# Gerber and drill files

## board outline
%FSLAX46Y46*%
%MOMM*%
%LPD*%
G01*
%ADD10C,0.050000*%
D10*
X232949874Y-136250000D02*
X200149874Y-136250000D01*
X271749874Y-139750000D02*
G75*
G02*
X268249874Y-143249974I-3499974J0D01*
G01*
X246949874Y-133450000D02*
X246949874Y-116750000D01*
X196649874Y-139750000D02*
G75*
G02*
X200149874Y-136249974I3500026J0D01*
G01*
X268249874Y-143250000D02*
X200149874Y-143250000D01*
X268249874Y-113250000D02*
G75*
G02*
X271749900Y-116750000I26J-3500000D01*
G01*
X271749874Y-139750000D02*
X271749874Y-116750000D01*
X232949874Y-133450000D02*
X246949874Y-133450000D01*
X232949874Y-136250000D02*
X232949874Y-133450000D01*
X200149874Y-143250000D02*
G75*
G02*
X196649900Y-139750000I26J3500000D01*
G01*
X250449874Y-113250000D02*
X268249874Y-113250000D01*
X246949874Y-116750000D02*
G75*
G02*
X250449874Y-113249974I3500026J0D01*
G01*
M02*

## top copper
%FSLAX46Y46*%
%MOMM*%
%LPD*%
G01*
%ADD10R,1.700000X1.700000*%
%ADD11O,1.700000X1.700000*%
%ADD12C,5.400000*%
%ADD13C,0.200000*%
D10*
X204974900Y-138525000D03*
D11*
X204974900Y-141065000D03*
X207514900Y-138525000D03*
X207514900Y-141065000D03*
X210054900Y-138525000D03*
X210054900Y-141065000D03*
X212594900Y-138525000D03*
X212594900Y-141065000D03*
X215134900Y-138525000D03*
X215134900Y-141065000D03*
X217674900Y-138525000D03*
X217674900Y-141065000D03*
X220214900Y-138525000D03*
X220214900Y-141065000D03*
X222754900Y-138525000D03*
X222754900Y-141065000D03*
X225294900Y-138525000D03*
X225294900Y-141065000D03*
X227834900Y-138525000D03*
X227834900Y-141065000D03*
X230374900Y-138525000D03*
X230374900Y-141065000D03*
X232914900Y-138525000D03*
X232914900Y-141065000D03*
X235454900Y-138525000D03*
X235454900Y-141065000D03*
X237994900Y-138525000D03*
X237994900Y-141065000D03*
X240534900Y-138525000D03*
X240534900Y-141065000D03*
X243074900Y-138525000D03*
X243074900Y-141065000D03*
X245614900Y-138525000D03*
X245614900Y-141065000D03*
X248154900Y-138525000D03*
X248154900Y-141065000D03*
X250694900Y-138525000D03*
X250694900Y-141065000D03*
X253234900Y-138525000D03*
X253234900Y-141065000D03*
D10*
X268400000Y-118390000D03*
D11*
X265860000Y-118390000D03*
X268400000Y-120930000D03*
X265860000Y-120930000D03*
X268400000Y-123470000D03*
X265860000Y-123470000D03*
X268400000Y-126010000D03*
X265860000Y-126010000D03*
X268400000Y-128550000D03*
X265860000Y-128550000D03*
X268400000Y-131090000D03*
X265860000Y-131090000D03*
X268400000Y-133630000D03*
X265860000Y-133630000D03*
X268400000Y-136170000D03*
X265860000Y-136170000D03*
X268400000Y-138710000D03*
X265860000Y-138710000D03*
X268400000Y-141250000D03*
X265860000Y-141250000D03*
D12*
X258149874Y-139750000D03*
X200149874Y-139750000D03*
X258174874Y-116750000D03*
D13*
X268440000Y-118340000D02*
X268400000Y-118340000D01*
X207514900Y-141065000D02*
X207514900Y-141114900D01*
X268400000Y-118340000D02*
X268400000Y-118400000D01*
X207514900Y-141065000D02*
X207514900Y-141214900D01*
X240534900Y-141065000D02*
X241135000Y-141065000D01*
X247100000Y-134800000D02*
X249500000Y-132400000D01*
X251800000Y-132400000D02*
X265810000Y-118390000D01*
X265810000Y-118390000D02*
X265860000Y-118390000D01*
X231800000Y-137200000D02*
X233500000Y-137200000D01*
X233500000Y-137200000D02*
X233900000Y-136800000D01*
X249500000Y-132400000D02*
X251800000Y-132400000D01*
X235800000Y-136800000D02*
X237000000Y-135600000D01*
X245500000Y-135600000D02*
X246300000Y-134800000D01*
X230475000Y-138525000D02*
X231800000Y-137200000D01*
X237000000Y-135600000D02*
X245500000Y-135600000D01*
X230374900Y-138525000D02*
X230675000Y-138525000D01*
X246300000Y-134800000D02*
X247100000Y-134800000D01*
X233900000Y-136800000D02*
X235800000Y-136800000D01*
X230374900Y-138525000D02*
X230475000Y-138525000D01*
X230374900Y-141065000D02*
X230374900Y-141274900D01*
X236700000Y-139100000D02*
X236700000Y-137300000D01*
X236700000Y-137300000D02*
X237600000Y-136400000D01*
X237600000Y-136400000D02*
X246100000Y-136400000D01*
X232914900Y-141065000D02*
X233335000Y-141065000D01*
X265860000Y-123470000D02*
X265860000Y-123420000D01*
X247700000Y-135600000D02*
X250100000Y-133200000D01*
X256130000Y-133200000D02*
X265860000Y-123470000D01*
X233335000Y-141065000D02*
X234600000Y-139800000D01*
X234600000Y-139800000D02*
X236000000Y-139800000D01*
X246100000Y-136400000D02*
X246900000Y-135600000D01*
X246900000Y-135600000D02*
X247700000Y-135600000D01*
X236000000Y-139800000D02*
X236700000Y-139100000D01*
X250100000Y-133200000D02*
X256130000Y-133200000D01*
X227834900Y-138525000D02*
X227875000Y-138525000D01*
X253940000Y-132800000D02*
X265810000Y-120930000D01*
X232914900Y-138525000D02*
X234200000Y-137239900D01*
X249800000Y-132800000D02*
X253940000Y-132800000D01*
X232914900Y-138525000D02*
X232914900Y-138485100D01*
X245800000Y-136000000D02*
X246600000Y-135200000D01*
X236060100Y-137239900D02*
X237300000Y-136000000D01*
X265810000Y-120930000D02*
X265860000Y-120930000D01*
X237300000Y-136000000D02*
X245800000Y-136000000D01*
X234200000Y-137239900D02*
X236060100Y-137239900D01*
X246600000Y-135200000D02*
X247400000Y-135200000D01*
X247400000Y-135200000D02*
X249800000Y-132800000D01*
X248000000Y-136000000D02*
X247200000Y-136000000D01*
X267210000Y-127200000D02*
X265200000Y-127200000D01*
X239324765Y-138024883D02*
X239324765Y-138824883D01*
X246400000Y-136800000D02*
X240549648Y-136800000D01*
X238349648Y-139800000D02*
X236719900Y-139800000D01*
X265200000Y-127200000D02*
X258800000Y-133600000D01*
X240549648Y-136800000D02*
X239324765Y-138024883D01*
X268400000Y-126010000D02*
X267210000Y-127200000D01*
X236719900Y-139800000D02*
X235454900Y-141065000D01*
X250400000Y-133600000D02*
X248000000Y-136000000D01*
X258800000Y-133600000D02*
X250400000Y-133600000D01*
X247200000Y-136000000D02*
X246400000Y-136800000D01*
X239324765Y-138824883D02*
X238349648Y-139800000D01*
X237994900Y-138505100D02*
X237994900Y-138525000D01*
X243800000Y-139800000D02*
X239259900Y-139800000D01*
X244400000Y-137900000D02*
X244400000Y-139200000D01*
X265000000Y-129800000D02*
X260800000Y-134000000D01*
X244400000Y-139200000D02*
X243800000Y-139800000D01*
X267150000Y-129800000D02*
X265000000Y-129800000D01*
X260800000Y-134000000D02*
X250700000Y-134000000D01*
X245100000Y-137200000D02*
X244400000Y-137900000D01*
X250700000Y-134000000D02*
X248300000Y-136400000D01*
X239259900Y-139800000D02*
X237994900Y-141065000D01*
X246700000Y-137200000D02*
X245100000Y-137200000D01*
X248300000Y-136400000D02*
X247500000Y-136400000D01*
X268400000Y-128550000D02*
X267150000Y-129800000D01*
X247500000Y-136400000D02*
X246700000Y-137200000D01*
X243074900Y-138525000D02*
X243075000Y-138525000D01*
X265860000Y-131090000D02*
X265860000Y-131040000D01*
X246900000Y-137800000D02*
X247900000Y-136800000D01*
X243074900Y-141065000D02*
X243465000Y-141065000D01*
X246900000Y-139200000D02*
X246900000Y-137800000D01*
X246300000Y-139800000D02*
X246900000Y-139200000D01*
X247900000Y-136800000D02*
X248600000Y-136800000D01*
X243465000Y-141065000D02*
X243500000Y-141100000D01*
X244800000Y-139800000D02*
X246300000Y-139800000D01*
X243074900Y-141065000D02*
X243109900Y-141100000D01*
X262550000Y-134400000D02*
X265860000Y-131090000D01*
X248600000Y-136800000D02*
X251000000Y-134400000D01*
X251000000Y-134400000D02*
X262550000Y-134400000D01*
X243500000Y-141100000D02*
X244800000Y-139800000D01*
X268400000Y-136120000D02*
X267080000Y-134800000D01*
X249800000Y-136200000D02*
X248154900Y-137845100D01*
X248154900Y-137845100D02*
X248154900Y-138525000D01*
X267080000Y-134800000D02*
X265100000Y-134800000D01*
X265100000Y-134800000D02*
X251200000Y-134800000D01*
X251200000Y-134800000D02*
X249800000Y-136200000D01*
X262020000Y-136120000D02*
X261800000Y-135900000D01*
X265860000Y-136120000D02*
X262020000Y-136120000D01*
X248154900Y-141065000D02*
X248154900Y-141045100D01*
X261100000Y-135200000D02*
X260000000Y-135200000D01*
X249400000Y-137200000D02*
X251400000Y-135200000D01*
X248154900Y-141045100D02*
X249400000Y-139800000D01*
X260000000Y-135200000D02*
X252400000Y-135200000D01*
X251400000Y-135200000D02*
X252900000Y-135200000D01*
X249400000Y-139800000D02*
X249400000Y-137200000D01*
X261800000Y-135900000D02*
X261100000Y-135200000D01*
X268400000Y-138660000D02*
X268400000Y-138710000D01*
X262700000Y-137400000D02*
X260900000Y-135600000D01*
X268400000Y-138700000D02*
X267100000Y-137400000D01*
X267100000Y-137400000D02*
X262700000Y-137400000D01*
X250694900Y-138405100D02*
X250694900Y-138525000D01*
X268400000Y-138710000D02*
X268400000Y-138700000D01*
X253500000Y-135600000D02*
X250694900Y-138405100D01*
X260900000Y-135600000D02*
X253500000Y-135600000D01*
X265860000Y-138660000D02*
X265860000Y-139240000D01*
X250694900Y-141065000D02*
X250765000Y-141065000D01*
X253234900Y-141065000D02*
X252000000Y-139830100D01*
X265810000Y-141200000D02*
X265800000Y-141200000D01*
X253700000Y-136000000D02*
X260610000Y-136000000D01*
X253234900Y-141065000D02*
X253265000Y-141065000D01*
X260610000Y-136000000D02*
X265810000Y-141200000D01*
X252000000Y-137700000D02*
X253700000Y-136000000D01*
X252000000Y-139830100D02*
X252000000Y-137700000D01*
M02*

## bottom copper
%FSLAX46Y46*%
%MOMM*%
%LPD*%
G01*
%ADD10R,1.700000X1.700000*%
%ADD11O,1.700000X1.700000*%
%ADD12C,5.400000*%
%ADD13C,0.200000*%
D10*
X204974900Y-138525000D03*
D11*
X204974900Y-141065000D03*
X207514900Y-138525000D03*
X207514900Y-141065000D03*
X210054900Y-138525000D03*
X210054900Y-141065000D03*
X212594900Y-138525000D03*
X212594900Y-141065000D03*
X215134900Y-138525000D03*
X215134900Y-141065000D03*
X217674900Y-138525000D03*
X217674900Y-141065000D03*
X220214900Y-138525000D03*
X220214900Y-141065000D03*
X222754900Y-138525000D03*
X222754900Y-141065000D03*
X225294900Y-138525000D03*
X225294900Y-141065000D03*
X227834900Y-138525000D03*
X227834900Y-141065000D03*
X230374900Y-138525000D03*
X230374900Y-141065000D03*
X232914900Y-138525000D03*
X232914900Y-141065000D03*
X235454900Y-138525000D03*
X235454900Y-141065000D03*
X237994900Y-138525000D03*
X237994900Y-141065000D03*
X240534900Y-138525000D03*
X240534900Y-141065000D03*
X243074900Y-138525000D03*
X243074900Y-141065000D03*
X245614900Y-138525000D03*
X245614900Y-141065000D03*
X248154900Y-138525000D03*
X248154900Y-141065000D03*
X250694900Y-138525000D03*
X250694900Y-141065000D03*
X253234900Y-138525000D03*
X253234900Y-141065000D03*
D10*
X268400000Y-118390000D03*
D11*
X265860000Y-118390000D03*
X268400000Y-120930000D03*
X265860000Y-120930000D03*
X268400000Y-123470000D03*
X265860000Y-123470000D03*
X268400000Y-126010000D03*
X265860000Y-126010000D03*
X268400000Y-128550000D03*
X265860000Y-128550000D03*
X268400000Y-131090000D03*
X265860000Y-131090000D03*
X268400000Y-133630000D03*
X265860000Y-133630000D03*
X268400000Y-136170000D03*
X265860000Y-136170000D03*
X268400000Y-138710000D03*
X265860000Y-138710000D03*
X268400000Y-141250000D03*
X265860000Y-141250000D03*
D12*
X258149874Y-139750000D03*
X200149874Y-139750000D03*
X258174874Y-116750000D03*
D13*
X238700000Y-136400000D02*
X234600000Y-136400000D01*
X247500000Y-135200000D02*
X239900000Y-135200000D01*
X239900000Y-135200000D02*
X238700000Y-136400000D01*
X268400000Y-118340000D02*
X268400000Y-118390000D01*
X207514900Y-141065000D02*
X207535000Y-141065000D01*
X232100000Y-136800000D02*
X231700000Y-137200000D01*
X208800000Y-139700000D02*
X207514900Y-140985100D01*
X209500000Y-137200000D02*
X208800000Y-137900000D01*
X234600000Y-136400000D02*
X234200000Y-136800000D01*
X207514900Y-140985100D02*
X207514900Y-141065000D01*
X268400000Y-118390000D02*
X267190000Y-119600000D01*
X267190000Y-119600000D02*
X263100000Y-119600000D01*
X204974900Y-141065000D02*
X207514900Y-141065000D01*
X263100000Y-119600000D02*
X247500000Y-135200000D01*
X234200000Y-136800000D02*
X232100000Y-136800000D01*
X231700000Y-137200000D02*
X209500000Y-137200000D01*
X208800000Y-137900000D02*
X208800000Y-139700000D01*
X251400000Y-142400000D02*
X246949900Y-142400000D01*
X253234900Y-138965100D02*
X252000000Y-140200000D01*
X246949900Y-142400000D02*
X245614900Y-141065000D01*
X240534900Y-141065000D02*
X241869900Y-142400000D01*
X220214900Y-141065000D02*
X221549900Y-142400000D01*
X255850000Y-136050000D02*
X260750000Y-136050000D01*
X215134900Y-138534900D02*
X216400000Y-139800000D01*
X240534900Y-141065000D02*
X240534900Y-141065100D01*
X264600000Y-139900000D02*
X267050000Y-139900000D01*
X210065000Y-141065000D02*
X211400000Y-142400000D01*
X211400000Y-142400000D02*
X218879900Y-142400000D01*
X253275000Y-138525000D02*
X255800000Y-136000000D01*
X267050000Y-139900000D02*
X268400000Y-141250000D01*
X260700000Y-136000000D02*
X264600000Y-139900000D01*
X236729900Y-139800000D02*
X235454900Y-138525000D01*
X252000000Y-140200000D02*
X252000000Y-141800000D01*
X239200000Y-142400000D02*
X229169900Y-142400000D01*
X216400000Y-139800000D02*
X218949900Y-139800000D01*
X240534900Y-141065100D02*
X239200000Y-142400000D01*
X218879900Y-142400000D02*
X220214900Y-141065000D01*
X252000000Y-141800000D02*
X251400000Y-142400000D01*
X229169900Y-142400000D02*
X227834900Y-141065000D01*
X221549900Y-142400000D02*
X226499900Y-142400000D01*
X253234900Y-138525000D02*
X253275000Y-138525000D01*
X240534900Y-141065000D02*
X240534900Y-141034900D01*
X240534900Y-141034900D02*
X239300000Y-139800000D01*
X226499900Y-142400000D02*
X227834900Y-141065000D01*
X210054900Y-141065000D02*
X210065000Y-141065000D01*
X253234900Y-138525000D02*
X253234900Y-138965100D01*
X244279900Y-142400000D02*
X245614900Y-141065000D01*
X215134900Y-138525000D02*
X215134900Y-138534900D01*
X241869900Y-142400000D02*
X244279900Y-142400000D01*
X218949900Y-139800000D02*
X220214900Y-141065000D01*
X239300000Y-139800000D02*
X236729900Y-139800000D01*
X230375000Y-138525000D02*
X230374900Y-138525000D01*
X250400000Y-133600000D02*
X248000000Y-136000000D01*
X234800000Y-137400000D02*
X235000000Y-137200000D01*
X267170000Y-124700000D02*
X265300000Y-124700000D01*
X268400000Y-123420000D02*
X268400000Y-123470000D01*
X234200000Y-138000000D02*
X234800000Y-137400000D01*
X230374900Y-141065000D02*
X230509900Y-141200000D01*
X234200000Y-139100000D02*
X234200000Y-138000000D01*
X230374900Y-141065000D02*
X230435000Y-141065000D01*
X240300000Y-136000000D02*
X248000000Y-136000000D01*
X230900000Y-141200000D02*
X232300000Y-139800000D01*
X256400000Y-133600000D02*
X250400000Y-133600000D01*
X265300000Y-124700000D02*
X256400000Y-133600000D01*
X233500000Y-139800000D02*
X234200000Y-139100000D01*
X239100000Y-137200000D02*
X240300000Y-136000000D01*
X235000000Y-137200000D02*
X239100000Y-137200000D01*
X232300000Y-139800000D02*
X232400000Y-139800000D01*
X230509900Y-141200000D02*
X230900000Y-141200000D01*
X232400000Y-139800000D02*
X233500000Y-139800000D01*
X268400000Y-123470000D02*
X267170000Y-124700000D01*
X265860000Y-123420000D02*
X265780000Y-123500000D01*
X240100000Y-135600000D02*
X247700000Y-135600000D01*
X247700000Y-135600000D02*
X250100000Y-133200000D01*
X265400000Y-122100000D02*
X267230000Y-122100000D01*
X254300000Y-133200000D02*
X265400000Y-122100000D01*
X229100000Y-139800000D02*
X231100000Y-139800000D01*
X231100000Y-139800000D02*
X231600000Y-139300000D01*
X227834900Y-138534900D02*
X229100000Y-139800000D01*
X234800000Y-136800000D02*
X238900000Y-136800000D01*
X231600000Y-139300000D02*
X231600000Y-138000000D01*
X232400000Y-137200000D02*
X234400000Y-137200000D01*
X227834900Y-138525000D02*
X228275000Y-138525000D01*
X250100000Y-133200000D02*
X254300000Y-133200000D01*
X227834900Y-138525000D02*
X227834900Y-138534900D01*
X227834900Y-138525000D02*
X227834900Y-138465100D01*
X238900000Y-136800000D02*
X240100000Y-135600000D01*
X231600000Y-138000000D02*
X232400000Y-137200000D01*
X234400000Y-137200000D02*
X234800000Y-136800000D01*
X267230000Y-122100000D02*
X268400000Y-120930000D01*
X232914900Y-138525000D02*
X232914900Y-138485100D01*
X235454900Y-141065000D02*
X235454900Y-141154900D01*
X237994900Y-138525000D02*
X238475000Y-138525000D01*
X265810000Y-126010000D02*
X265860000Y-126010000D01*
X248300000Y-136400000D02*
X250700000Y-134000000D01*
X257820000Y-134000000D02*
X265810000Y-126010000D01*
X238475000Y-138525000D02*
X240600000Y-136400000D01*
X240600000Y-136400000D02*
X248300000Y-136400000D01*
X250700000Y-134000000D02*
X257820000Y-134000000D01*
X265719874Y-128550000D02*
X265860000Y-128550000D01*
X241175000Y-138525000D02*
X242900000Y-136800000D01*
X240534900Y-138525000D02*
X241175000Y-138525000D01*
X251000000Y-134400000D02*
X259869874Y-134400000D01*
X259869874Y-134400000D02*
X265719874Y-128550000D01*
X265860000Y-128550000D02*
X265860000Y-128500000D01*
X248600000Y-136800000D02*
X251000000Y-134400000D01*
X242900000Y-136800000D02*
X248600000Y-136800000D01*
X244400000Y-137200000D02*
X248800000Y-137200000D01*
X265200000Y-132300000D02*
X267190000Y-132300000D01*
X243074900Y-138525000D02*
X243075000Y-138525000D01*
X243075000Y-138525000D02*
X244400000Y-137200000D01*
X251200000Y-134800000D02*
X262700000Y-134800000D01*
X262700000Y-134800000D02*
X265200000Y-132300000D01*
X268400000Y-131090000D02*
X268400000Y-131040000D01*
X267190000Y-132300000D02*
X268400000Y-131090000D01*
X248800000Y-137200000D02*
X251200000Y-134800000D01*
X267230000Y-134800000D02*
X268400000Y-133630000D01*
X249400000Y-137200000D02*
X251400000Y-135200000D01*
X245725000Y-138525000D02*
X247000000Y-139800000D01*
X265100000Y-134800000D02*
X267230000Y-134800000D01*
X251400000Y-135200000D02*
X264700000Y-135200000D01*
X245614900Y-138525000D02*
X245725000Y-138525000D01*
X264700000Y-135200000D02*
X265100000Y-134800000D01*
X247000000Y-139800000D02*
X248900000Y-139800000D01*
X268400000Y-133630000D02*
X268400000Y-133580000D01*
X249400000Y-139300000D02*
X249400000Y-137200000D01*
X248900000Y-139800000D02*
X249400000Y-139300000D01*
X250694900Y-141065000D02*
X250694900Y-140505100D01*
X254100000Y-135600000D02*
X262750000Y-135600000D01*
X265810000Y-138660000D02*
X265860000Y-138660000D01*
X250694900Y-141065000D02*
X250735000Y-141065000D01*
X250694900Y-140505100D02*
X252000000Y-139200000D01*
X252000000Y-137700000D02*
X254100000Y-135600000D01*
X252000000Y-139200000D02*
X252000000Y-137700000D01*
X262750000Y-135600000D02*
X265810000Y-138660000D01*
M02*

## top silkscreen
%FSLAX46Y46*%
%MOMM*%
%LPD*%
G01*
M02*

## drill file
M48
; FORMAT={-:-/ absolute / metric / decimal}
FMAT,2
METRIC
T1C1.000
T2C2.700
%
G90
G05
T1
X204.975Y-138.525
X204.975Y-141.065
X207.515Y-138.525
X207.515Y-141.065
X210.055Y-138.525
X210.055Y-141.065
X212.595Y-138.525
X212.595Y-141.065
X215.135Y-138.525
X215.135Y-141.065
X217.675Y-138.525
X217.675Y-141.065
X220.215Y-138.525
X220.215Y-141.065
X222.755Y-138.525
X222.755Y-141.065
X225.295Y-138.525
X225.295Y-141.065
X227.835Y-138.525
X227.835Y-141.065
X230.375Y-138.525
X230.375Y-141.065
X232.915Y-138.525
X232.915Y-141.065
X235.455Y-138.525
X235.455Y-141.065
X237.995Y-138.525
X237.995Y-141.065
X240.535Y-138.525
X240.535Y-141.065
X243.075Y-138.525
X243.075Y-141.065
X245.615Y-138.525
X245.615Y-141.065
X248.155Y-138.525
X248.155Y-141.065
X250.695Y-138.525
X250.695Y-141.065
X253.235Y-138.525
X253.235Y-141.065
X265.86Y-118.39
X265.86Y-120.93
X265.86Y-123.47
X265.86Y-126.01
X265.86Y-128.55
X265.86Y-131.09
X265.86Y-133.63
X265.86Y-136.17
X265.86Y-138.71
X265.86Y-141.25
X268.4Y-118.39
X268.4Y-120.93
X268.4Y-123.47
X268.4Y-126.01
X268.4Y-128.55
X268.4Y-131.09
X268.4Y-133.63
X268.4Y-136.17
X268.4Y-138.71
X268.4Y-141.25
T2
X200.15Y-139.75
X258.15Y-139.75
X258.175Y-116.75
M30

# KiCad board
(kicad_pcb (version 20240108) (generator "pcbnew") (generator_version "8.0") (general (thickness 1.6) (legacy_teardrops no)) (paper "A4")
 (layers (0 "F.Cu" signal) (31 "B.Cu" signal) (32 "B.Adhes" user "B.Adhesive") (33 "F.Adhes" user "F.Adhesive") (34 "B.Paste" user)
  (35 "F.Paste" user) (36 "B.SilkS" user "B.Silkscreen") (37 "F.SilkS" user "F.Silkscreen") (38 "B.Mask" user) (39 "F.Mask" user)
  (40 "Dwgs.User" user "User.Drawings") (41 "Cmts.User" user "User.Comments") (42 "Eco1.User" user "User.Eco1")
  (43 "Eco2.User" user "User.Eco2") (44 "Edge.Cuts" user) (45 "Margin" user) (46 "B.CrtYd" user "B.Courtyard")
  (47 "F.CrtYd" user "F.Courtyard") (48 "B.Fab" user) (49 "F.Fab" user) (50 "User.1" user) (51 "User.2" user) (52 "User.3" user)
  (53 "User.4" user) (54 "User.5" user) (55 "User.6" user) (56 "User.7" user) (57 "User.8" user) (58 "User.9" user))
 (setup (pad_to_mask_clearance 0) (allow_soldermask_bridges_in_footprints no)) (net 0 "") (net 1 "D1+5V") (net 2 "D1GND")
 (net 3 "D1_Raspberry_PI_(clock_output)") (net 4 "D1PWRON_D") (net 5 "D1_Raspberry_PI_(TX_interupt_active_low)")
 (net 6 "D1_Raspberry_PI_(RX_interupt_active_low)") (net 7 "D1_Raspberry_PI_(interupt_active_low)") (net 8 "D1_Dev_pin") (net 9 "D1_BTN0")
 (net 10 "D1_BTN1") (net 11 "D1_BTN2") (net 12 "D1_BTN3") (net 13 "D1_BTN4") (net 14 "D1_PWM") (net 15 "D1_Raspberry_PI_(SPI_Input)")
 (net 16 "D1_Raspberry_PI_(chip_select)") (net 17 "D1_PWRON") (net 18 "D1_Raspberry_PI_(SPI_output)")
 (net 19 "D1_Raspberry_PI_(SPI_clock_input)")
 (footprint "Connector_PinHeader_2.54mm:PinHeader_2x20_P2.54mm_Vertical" (layer "B.Cu") (at 204.9749 138.525 -90)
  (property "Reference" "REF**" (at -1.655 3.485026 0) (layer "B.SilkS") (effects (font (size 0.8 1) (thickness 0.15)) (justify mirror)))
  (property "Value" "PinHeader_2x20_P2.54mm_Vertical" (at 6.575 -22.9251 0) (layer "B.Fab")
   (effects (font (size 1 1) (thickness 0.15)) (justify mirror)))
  (pad "1" thru_hole rect (at 0 0 270) (size 1.7 1.7) (drill 1) (layers "*.Cu" "*.Mask") (remove_unused_layers no))
  (pad "2" thru_hole oval (at 2.54 0 270) (size 1.7 1.7) (drill 1) (layers "*.Cu" "*.Mask") (remove_unused_layers no) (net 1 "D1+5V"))
  (pad "3" thru_hole oval (at 0 -2.54 270) (size 1.7 1.7) (drill 1) (layers "*.Cu" "*.Mask") (remove_unused_layers no))
  (pad "4" thru_hole oval (at 2.54 -2.54 270) (size 1.7 1.7) (drill 1) (layers "*.Cu" "*.Mask") (remove_unused_layers no) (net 1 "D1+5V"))
  (pad "5" thru_hole oval (at 0 -5.08 270) (size 1.7 1.7) (drill 1) (layers "*.Cu" "*.Mask") (remove_unused_layers no))
  (pad "6" thru_hole oval (at 2.54 -5.08 270) (size 1.7 1.7) (drill 1) (layers "*.Cu" "*.Mask") (remove_unused_layers no) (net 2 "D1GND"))
  (pad "7" thru_hole oval (at 0 -7.62 270) (size 1.7 1.7) (drill 1) (layers "*.Cu" "*.Mask") (remove_unused_layers no))
  (pad "8" thru_hole oval (at 2.54 -7.62 270) (size 1.7 1.7) (drill 1) (layers "*.Cu" "*.Mask") (remove_unused_layers no))
  (pad "9" thru_hole oval (at 0 -10.16 270) (size 1.7 1.7) (drill 1) (layers "*.Cu" "*.Mask") (remove_unused_layers no) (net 2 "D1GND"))
  (pad "10" thru_hole oval (at 2.54 -10.16 270) (size 1.7 1.7) (drill 1) (layers "*.Cu" "*.Mask") (remove_unused_layers no))
  (pad "11" thru_hole oval (at 0 -12.7 270) (size 1.7 1.7) (drill 1) (layers "*.Cu" "*.Mask") (remove_unused_layers no))
  (pad "12" thru_hole oval (at 2.54 -12.7 270) (size 1.7 1.7) (drill 1) (layers "*.Cu" "*.Mask") (remove_unused_layers no))
  (pad "13" thru_hole oval (at 0 -15.24 270) (size 1.7 1.7) (drill 1) (layers "*.Cu" "*.Mask") (remove_unused_layers no))
  (pad "14" thru_hole oval (at 2.54 -15.24 270) (size 1.7 1.7) (drill 1) (layers "*.Cu" "*.Mask") (remove_unused_layers no) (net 2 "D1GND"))
  (pad "15" thru_hole oval (at 0 -17.78 270) (size 1.7 1.7) (drill 1) (layers "*.Cu" "*.Mask") (remove_unused_layers no))
  (pad "16" thru_hole oval (at 2.54 -17.78 270) (size 1.7 1.7) (drill 1) (layers "*.Cu" "*.Mask") (remove_unused_layers no))
  (pad "17" thru_hole oval (at 0 -20.32 270) (size 1.7 1.7) (drill 1) (layers "*.Cu" "*.Mask") (remove_unused_layers no))
  (pad "18" thru_hole oval (at 2.54 -20.32 270) (size 1.7 1.7) (drill 1) (layers "*.Cu" "*.Mask") (remove_unused_layers no))
  (pad "19" thru_hole oval (at 0 -22.86 270) (size 1.7 1.7) (drill 1) (layers "*.Cu" "*.Mask") (remove_unused_layers no)
   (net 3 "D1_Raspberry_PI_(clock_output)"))
  (pad "20" thru_hole oval (at 2.54 -22.86 270) (size 1.7 1.7) (drill 1) (layers "*.Cu" "*.Mask") (remove_unused_layers no) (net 2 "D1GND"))
  (pad "21" thru_hole oval (at 0 -25.4 270) (size 1.7 1.7) (drill 1) (layers "*.Cu" "*.Mask") (remove_unused_layers no) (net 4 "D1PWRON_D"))
  (pad "22" thru_hole oval (at 2.54 -25.4 270) (size 1.7 1.7) (drill 1) (layers "*.Cu" "*.Mask") (remove_unused_layers no)
   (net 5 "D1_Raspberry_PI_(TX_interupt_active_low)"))
  (pad "23" thru_hole oval (at 0 -27.94 270) (size 1.7 1.7) (drill 1) (layers "*.Cu" "*.Mask") (remove_unused_layers no)
   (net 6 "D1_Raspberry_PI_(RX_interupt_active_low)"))
  (pad "24" thru_hole oval (at 2.54 -27.94 270) (size 1.7 1.7) (drill 1) (layers "*.Cu" "*.Mask") (remove_unused_layers no)
   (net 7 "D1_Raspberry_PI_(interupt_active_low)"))
  (pad "25" thru_hole oval (at 0 -30.48 270) (size 1.7 1.7) (drill 1) (layers "*.Cu" "*.Mask") (remove_unused_layers no) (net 2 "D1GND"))
  (pad "26" thru_hole oval (at 2.54 -30.48 270) (size 1.7 1.7) (drill 1) (layers "*.Cu" "*.Mask") (remove_unused_layers no)
   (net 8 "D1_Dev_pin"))
  (pad "27" thru_hole oval (at 0 -33.02 270) (size 1.7 1.7) (drill 1) (layers "*.Cu" "*.Mask") (remove_unused_layers no) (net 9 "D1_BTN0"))
  (pad "28" thru_hole oval (at 2.54 -33.02 270) (size 1.7 1.7) (drill 1) (layers "*.Cu" "*.Mask") (remove_unused_layers no)
   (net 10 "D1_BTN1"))
  (pad "29" thru_hole oval (at 0 -35.56 270) (size 1.7 1.7) (drill 1) (layers "*.Cu" "*.Mask") (remove_unused_layers no) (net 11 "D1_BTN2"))
  (pad "30" thru_hole oval (at 2.54 -35.56 270) (size 1.7 1.7) (drill 1) (layers "*.Cu" "*.Mask") (remove_unused_layers no) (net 2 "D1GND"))
  (pad "31" thru_hole oval (at 0 -38.1 270) (size 1.7 1.7) (drill 1) (layers "*.Cu" "*.Mask") (remove_unused_layers no) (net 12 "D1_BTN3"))
  (pad "32" thru_hole oval (at 2.54 -38.1 270) (size 1.7 1.7) (drill 1) (layers "*.Cu" "*.Mask") (remove_unused_layers no)
   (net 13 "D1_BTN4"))
  (pad "33" thru_hole oval (at 0 -40.64 270) (size 1.7 1.7) (drill 1) (layers "*.Cu" "*.Mask") (remove_unused_layers no) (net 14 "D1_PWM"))
  (pad "34" thru_hole oval (at 2.54 -40.64 270) (size 1.7 1.7) (drill 1) (layers "*.Cu" "*.Mask") (remove_unused_layers no) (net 2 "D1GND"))
  (pad "35" thru_hole oval (at 0 -43.18 270) (size 1.7 1.7) (drill 1) (layers "*.Cu" "*.Mask") (remove_unused_layers no)
   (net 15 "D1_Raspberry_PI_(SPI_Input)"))
  (pad "36" thru_hole oval (at 2.54 -43.18 270) (size 1.7 1.7) (drill 1) (layers "*.Cu" "*.Mask") (remove_unused_layers no)
   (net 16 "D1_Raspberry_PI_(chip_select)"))
  (pad "37" thru_hole oval (at 0 -45.72 270) (size 1.7 1.7) (drill 1) (layers "*.Cu" "*.Mask") (remove_unused_layers no) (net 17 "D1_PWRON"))
  (pad "38" thru_hole oval (at 2.54 -45.72 270) (size 1.7 1.7) (drill 1) (layers "*.Cu" "*.Mask") (remove_unused_layers no)
   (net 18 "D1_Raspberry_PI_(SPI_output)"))
  (pad "39" thru_hole oval (at 0 -48.26 270) (size 1.7 1.7) (drill 1) (layers "*.Cu" "*.Mask") (remove_unused_layers no) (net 2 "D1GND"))
  (pad "40" thru_hole oval (at 2.54 -48.26 270) (size 1.7 1.7) (drill 1) (layers "*.Cu" "*.Mask") (remove_unused_layers no)
   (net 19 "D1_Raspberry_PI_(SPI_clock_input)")))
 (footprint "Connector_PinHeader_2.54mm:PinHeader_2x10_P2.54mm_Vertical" (layer "B.Cu") (at 268.4 118.39 180)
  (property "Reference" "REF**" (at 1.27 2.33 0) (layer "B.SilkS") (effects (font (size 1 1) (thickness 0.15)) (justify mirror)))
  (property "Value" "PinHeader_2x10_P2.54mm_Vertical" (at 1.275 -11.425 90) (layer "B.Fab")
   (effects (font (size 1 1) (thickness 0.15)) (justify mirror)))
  (pad "1" thru_hole rect (at 0 0 180) (size 1.7 1.7) (drill 1) (layers "*.Cu" "*.Mask") (remove_unused_layers no) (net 1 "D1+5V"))
  (pad "2" thru_hole oval (at 2.54 0 180) (size 1.7 1.7) (drill 1) (layers "*.Cu" "*.Mask") (remove_unused_layers no) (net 4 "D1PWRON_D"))
  (pad "3" thru_hole oval (at 0 -2.54 180) (size 1.7 1.7) (drill 1) (layers "*.Cu" "*.Mask") (remove_unused_layers no)
   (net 3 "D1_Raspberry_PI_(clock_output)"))
  (pad "4" thru_hole oval (at 2.54 -2.54 180) (size 1.7 1.7) (drill 1) (layers "*.Cu" "*.Mask") (remove_unused_layers no)
   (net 6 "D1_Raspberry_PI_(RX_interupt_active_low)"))
  (pad "5" thru_hole oval (at 0 -5.08 180) (size 1.7 1.7) (drill 1) (layers "*.Cu" "*.Mask") (remove_unused_layers no)
   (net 5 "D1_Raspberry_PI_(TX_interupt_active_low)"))
  (pad "6" thru_hole oval (at 2.54 -5.08 180) (size 1.7 1.7) (drill 1) (layers "*.Cu" "*.Mask") (remove_unused_layers no)
   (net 7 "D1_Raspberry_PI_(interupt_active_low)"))
  (pad "7" thru_hole oval (at 0 -7.62 180) (size 1.7 1.7) (drill 1) (layers "*.Cu" "*.Mask") (remove_unused_layers no) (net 8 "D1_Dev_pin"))
  (pad "8" thru_hole oval (at 2.54 -7.62 180) (size 1.7 1.7) (drill 1) (layers "*.Cu" "*.Mask") (remove_unused_layers no) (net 9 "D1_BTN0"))
  (pad "9" thru_hole oval (at 0 -10.16 180) (size 1.7 1.7) (drill 1) (layers "*.Cu" "*.Mask") (remove_unused_layers no) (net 10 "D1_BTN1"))
  (pad "10" thru_hole oval (at 2.54 -10.16 180) (size 1.7 1.7) (drill 1) (layers "*.Cu" "*.Mask") (remove_unused_layers no)
   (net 11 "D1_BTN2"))
  (pad "11" thru_hole oval (at 0 -12.7 180) (size 1.7 1.7) (drill 1) (layers "*.Cu" "*.Mask") (remove_unused_layers no) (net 12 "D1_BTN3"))
  (pad "12" thru_hole oval (at 2.54 -12.7 180) (size 1.7 1.7) (drill 1) (layers "*.Cu" "*.Mask") (remove_unused_layers no)
   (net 13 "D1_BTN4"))
  (pad "13" thru_hole oval (at 0 -15.24 180) (size 1.7 1.7) (drill 1) (layers "*.Cu" "*.Mask") (remove_unused_layers no) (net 14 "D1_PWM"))
  (pad "14" thru_hole oval (at 2.54 -15.24 180) (size 1.7 1.7) (drill 1) (layers "*.Cu" "*.Mask") (remove_unused_layers no))
  (pad "15" thru_hole oval (at 0 -17.78 180) (size 1.7 1.7) (drill 1) (layers "*.Cu" "*.Mask") (remove_unused_layers no)
   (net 15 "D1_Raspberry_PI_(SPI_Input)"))
  (pad "16" thru_hole oval (at 2.54 -17.78 180) (size 1.7 1.7) (drill 1) (layers "*.Cu" "*.Mask") (remove_unused_layers no)
   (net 16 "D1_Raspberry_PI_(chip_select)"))
  (pad "17" thru_hole oval (at 0 -20.32 180) (size 1.7 1.7) (drill 1) (layers "*.Cu" "*.Mask") (remove_unused_layers no) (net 17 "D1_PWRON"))
  (pad "18" thru_hole oval (at 2.54 -20.32 180) (size 1.7 1.7) (drill 1) (layers "*.Cu" "*.Mask") (remove_unused_layers no)
   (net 18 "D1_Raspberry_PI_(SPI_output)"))
  (pad "19" thru_hole oval (at 0 -22.86 180) (size 1.7 1.7) (drill 1) (layers "*.Cu" "*.Mask") (remove_unused_layers no) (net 2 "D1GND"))
  (pad "20" thru_hole oval (at 2.54 -22.86 180) (size 1.7 1.7) (drill 1) (layers "*.Cu" "*.Mask") (remove_unused_layers no)
   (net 19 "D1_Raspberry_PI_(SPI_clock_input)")))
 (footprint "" (layer "B.Cu") (at 258.149874 139.75 180)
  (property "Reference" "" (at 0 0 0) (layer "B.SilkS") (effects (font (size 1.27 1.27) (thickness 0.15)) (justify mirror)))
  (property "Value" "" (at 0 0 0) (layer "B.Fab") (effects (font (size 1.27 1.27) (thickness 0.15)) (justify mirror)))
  (pad "1" thru_hole circle (at 0 0 180) (size 5.4 5.4) (drill 2.7) (layers "*.Cu" "*.Mask") (remove_unused_layers no)))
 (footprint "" (layer "B.Cu") (at 200.149874 139.75 180)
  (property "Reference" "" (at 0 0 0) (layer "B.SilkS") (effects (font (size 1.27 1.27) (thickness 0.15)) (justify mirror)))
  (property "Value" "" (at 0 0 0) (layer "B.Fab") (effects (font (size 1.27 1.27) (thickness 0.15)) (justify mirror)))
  (pad "1" thru_hole circle (at 0 0 180) (size 5.4 5.4) (drill 2.7) (layers "*.Cu" "*.Mask") (remove_unused_layers no)))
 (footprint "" (layer "B.Cu") (at 258.174874 116.75 180)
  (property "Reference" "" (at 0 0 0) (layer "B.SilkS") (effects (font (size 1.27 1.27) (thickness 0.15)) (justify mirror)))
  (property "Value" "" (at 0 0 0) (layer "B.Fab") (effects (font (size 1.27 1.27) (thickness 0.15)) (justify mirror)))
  (pad "1" thru_hole circle (at 0 0 180) (size 5.4 5.4) (drill 2.7) (layers "*.Cu" "*.Mask") (remove_unused_layers no)))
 (gr_line (start 232.949874 136.25) (end 200.149874 136.25) (stroke (width 0.05) (type default)) (layer "Edge.Cuts"))
 (gr_arc (start 271.749874 139.75) (mid 270.724748 142.224874) (end 268.249874 143.25) (stroke (width 0.05) (type default))
  (layer "Edge.Cuts"))
 (gr_line (start 246.949874 133.45) (end 246.949874 116.75) (stroke (width 0.05) (type default)) (layer "Edge.Cuts"))
 (gr_arc (start 196.649874 139.75) (mid 197.675 137.275126) (end 200.149874 136.25) (stroke (width 0.05) (type default)) (layer "Edge.Cuts"))
 (gr_line (start 268.249874 143.25) (end 200.149874 143.25) (stroke (width 0.05) (type default)) (layer "Edge.Cuts"))
 (gr_arc (start 268.249874 113.25) (mid 270.724748 114.275126) (end 271.749874 116.75) (stroke (width 0.05) (type default))
  (layer "Edge.Cuts"))
 (gr_line (start 271.749874 139.75) (end 271.749874 116.75) (stroke (width 0.05) (type default)) (layer "Edge.Cuts"))
 (gr_line (start 232.949874 133.45) (end 246.949874 133.45) (stroke (width 0.05) (type default)) (layer "Edge.Cuts"))
 (gr_line (start 232.949874 136.25) (end 232.949874 133.45) (stroke (width 0.05) (type default)) (layer "Edge.Cuts"))
 (gr_arc (start 200.149874 143.25) (mid 197.675 142.224874) (end 196.649874 139.75) (stroke (width 0.05) (type default)) (layer "Edge.Cuts"))
 (gr_line (start 250.449874 113.25) (end 268.249874 113.25) (stroke (width 0.05) (type default)) (layer "Edge.Cuts"))
 (gr_arc (start 246.949874 116.75) (mid 247.975 114.275126) (end 250.449874 113.25) (stroke (width 0.05) (type default)) (layer "Edge.Cuts"))
 (segment (start 268.44 118.34) (end 268.4 118.34) (width 0.2) (layer "F.Cu") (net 1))
 (segment (start 207.5149 141.065) (end 207.5149 141.1149) (width 0.2) (layer "F.Cu") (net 1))
 (segment (start 268.4 118.34) (end 268.4 118.4) (width 0.2) (layer "F.Cu") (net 1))
 (segment (start 207.5149 141.065) (end 207.5149 141.2149) (width 0.2) (layer "F.Cu") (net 1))
 (segment (start 238.7 136.4) (end 234.6 136.4) (width 0.2) (layer "B.Cu") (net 1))
 (segment (start 247.5 135.2) (end 239.9 135.2) (width 0.2) (layer "B.Cu") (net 1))
 (segment (start 239.9 135.2) (end 238.7 136.4) (width 0.2) (layer "B.Cu") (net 1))
 (segment (start 268.4 118.34) (end 268.4 118.39) (width 0.2) (layer "B.Cu") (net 1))
 (segment (start 207.5149 141.065) (end 207.535 141.065) (width 0.2) (layer "B.Cu") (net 1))
 (segment (start 232.1 136.8) (end 231.7 137.2) (width 0.2) (layer "B.Cu") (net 1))
 (segment (start 208.8 139.7) (end 207.5149 140.9851) (width 0.2) (layer "B.Cu") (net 1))
 (segment (start 209.5 137.2) (end 208.8 137.9) (width 0.2) (layer "B.Cu") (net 1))
 (segment (start 234.6 136.4) (end 234.2 136.8) (width 0.2) (layer "B.Cu") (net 1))
 (segment (start 207.5149 140.9851) (end 207.5149 141.065) (width 0.2) (layer "B.Cu") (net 1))
 (segment (start 268.4 118.39) (end 267.19 119.6) (width 0.2) (layer "B.Cu") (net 1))
 (segment (start 267.19 119.6) (end 263.1 119.6) (width 0.2) (layer "B.Cu") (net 1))
 (segment (start 204.9749 141.065) (end 207.5149 141.065) (width 0.2) (layer "B.Cu") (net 1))
 (segment (start 263.1 119.6) (end 247.5 135.2) (width 0.2) (layer "B.Cu") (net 1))
 (segment (start 234.2 136.8) (end 232.1 136.8) (width 0.2) (layer "B.Cu") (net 1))
 (segment (start 231.7 137.2) (end 209.5 137.2) (width 0.2) (layer "B.Cu") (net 1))
 (segment (start 208.8 137.9) (end 208.8 139.7) (width 0.2) (layer "B.Cu") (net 1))
 (segment (start 240.5349 141.065) (end 241.135 141.065) (width 0.2) (layer "F.Cu") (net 2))
 (segment (start 251.4 142.4) (end 246.9499 142.4) (width 0.2) (layer "B.Cu") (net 2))
 (segment (start 253.2349 138.9651) (end 252 140.2) (width 0.2) (layer "B.Cu") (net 2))
 (segment (start 246.9499 142.4) (end 245.6149 141.065) (width 0.2) (layer "B.Cu") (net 2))
 (segment (start 240.5349 141.065) (end 241.8699 142.4) (width 0.2) (layer "B.Cu") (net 2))
 (segment (start 220.2149 141.065) (end 221.5499 142.4) (width 0.2) (layer "B.Cu") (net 2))
 (segment (start 255.85 136.05) (end 260.75 136.05) (width 0.2) (layer "B.Cu") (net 2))
 (segment (start 215.1349 138.5349) (end 216.4 139.8) (width 0.2) (layer "B.Cu") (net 2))
 (segment (start 240.5349 141.065) (end 240.5349 141.0651) (width 0.2) (layer "B.Cu") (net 2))
 (segment (start 264.6 139.9) (end 267.05 139.9) (width 0.2) (layer "B.Cu") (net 2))
 (segment (start 210.065 141.065) (end 211.4 142.4) (width 0.2) (layer "B.Cu") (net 2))
 (segment (start 211.4 142.4) (end 218.8799 142.4) (width 0.2) (layer "B.Cu") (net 2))
 (segment (start 253.275 138.525) (end 255.8 136) (width 0.2) (layer "B.Cu") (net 2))
 (segment (start 267.05 139.9) (end 268.4 141.25) (width 0.2) (layer "B.Cu") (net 2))
 (segment (start 260.7 136) (end 264.6 139.9) (width 0.2) (layer "B.Cu") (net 2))
 (segment (start 236.7299 139.8) (end 235.4549 138.525) (width 0.2) (layer "B.Cu") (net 2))
 (segment (start 252 140.2) (end 252 141.8) (width 0.2) (layer "B.Cu") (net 2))
 (segment (start 239.2 142.4) (end 229.1699 142.4) (width 0.2) (layer "B.Cu") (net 2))
 (segment (start 216.4 139.8) (end 218.9499 139.8) (width 0.2) (layer "B.Cu") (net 2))
 (segment (start 240.5349 141.0651) (end 239.2 142.4) (width 0.2) (layer "B.Cu") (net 2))
 (segment (start 218.8799 142.4) (end 220.2149 141.065) (width 0.2) (layer "B.Cu") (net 2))
 (segment (start 252 141.8) (end 251.4 142.4) (width 0.2) (layer "B.Cu") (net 2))
 (segment (start 229.1699 142.4) (end 227.8349 141.065) (width 0.2) (layer "B.Cu") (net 2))
 (segment (start 221.5499 142.4) (end 226.4999 142.4) (width 0.2) (layer "B.Cu") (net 2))
 (segment (start 253.2349 138.525) (end 253.275 138.525) (width 0.2) (layer "B.Cu") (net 2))
 (segment (start 240.5349 141.065) (end 240.5349 141.0349) (width 0.2) (layer "B.Cu") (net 2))
 (segment (start 240.5349 141.0349) (end 239.3 139.8) (width 0.2) (layer "B.Cu") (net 2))
 (segment (start 226.4999 142.4) (end 227.8349 141.065) (width 0.2) (layer "B.Cu") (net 2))
 (segment (start 210.0549 141.065) (end 210.065 141.065) (width 0.2) (layer "B.Cu") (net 2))
 (segment (start 253.2349 138.525) (end 253.2349 138.9651) (width 0.2) (layer "B.Cu") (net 2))
 (segment (start 244.2799 142.4) (end 245.6149 141.065) (width 0.2) (layer "B.Cu") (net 2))
 (segment (start 215.1349 138.525) (end 215.1349 138.5349) (width 0.2) (layer "B.Cu") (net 2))
 (segment (start 241.8699 142.4) (end 244.2799 142.4) (width 0.2) (layer "B.Cu") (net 2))
 (segment (start 218.9499 139.8) (end 220.2149 141.065) (width 0.2) (layer "B.Cu") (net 2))
 (segment (start 239.3 139.8) (end 236.7299 139.8) (width 0.2) (layer "B.Cu") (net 2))
 (segment (start 247.1 134.8) (end 249.5 132.4) (width 0.2) (layer "F.Cu") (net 4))
 (segment (start 251.8 132.4) (end 265.81 118.39) (width 0.2) (layer "F.Cu") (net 4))
 (segment (start 265.81 118.39) (end 265.86 118.39) (width 0.2) (layer "F.Cu") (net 4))
 (segment (start 231.8 137.2) (end 233.5 137.2) (width 0.2) (layer "F.Cu") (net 4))
 (segment (start 233.5 137.2) (end 233.9 136.8) (width 0.2) (layer "F.Cu") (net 4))
 (segment (start 249.5 132.4) (end 251.8 132.4) (width 0.2) (layer "F.Cu") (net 4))
 (segment (start 235.8 136.8) (end 237 135.6) (width 0.2) (layer "F.Cu") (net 4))
 (segment (start 245.5 135.6) (end 246.3 134.8) (width 0.2) (layer "F.Cu") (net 4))
 (segment (start 230.475 138.525) (end 231.8 137.2) (width 0.2) (layer "F.Cu") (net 4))
 (segment (start 237 135.6) (end 245.5 135.6) (width 0.2) (layer "F.Cu") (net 4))
 (segment (start 230.3749 138.525) (end 230.675 138.525) (width 0.2) (layer "F.Cu") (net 4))
 (segment (start 246.3 134.8) (end 247.1 134.8) (width 0.2) (layer "F.Cu") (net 4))
 (segment (start 233.9 136.8) (end 235.8 136.8) (width 0.2) (layer "F.Cu") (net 4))
 (segment (start 230.3749 138.525) (end 230.475 138.525) (width 0.2) (layer "F.Cu") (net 4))
 (segment (start 230.375 138.525) (end 230.3749 138.525) (width 0.2) (layer "B.Cu") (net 4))
 (segment (start 230.3749 141.065) (end 230.3749 141.2749) (width 0.2) (layer "F.Cu") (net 5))
 (segment (start 250.4 133.6) (end 248 136) (width 0.2) (layer "B.Cu") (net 5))
 (segment (start 234.8 137.4) (end 235 137.2) (width 0.2) (layer "B.Cu") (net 5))
 (segment (start 267.17 124.7) (end 265.3 124.7) (width 0.2) (layer "B.Cu") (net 5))
 (segment (start 268.4 123.42) (end 268.4 123.47) (width 0.2) (layer "B.Cu") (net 5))
 (segment (start 234.2 138) (end 234.8 137.4) (width 0.2) (layer "B.Cu") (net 5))
 (segment (start 230.3749 141.065) (end 230.5099 141.2) (width 0.2) (layer "B.Cu") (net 5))
 (segment (start 234.2 139.1) (end 234.2 138) (width 0.2) (layer "B.Cu") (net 5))
 (segment (start 230.3749 141.065) (end 230.435 141.065) (width 0.2) (layer "B.Cu") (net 5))
 (segment (start 240.3 136) (end 248 136) (width 0.2) (layer "B.Cu") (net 5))
 (segment (start 230.9 141.2) (end 232.3 139.8) (width 0.2) (layer "B.Cu") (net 5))
 (segment (start 256.4 133.6) (end 250.4 133.6) (width 0.2) (layer "B.Cu") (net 5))
 (segment (start 265.3 124.7) (end 256.4 133.6) (width 0.2) (layer "B.Cu") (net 5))
 (segment (start 233.5 139.8) (end 234.2 139.1) (width 0.2) (layer "B.Cu") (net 5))
 (segment (start 239.1 137.2) (end 240.3 136) (width 0.2) (layer "B.Cu") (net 5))
 (segment (start 235 137.2) (end 239.1 137.2) (width 0.2) (layer "B.Cu") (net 5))
 (segment (start 232.3 139.8) (end 232.4 139.8) (width 0.2) (layer "B.Cu") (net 5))
 (segment (start 230.5099 141.2) (end 230.9 141.2) (width 0.2) (layer "B.Cu") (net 5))
 (segment (start 232.4 139.8) (end 233.5 139.8) (width 0.2) (layer "B.Cu") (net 5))
 (segment (start 268.4 123.47) (end 267.17 124.7) (width 0.2) (layer "B.Cu") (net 5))
 (segment (start 236.7 139.1) (end 236.7 137.3) (width 0.2) (layer "F.Cu") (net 7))
 (segment (start 236.7 137.3) (end 237.6 136.4) (width 0.2) (layer "F.Cu") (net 7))
 (segment (start 237.6 136.4) (end 246.1 136.4) (width 0.2) (layer "F.Cu") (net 7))
 (segment (start 232.9149 141.065) (end 233.335 141.065) (width 0.2) (layer "F.Cu") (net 7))
 (segment (start 265.86 123.47) (end 265.86 123.42) (width 0.2) (layer "F.Cu") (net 7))
 (segment (start 247.7 135.6) (end 250.1 133.2) (width 0.2) (layer "F.Cu") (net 7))
 (segment (start 256.13 133.2) (end 265.86 123.47) (width 0.2) (layer "F.Cu") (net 7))
 (segment (start 233.335 141.065) (end 234.6 139.8) (width 0.2) (layer "F.Cu") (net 7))
 (segment (start 234.6 139.8) (end 236 139.8) (width 0.2) (layer "F.Cu") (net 7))
 (segment (start 246.1 136.4) (end 246.9 135.6) (width 0.2) (layer "F.Cu") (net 7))
 (segment (start 246.9 135.6) (end 247.7 135.6) (width 0.2) (layer "F.Cu") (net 7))
 (segment (start 236 139.8) (end 236.7 139.1) (width 0.2) (layer "F.Cu") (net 7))
 (segment (start 250.1 133.2) (end 256.13 133.2) (width 0.2) (layer "F.Cu") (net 7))
 (segment (start 265.86 123.42) (end 265.78 123.5) (width 0.2) (layer "B.Cu") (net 7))
 (segment (start 227.8349 138.525) (end 227.875 138.525) (width 0.2) (layer "F.Cu") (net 3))
 (segment (start 240.1 135.6) (end 247.7 135.6) (width 0.2) (layer "B.Cu") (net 3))
 (segment (start 247.7 135.6) (end 250.1 133.2) (width 0.2) (layer "B.Cu") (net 3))
 (segment (start 265.4 122.1) (end 267.23 122.1) (width 0.2) (layer "B.Cu") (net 3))
 (segment (start 254.3 133.2) (end 265.4 122.1) (width 0.2) (layer "B.Cu") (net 3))
 (segment (start 229.1 139.8) (end 231.1 139.8) (width 0.2) (layer "B.Cu") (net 3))
 (segment (start 231.1 139.8) (end 231.6 139.3) (width 0.2) (layer "B.Cu") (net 3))
 (segment (start 227.8349 138.5349) (end 229.1 139.8) (width 0.2) (layer "B.Cu") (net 3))
 (segment (start 234.8 136.8) (end 238.9 136.8) (width 0.2) (layer "B.Cu") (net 3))
 (segment (start 231.6 139.3) (end 231.6 138) (width 0.2) (layer "B.Cu") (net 3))
 (segment (start 232.4 137.2) (end 234.4 137.2) (width 0.2) (layer "B.Cu") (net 3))
 (segment (start 227.8349 138.525) (end 228.275 138.525) (width 0.2) (layer "B.Cu") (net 3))
 (segment (start 250.1 133.2) (end 254.3 133.2) (width 0.2) (layer "B.Cu") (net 3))
 (segment (start 227.8349 138.525) (end 227.8349 138.5349) (width 0.2) (layer "B.Cu") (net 3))
 (segment (start 227.8349 138.525) (end 227.8349 138.4651) (width 0.2) (layer "B.Cu") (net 3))
 (segment (start 238.9 136.8) (end 240.1 135.6) (width 0.2) (layer "B.Cu") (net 3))
 (segment (start 231.6 138) (end 232.4 137.2) (width 0.2) (layer "B.Cu") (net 3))
 (segment (start 234.4 137.2) (end 234.8 136.8) (width 0.2) (layer "B.Cu") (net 3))
 (segment (start 267.23 122.1) (end 268.4 120.93) (width 0.2) (layer "B.Cu") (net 3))
 (segment (start 253.94 132.8) (end 265.81 120.93) (width 0.2) (layer "F.Cu") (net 6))
 (segment (start 232.9149 138.525) (end 234.2 137.2399) (width 0.2) (layer "F.Cu") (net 6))
 (segment (start 249.8 132.8) (end 253.94 132.8) (width 0.2) (layer "F.Cu") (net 6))
 (segment (start 232.9149 138.525) (end 232.9149 138.4851) (width 0.2) (layer "F.Cu") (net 6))
 (segment (start 245.8 136) (end 246.6 135.2) (width 0.2) (layer "F.Cu") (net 6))
 (segment (start 236.0601 137.2399) (end 237.3 136) (width 0.2) (layer "F.Cu") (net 6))
 (segment (start 265.81 120.93) (end 265.86 120.93) (width 0.2) (layer "F.Cu") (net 6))
 (segment (start 237.3 136) (end 245.8 136) (width 0.2) (layer "F.Cu") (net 6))
 (segment (start 234.2 137.2399) (end 236.0601 137.2399) (width 0.2) (layer "F.Cu") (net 6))
 (segment (start 246.6 135.2) (end 247.4 135.2) (width 0.2) (layer "F.Cu") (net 6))
 (segment (start 247.4 135.2) (end 249.8 132.8) (width 0.2) (layer "F.Cu") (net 6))
 (segment (start 232.9149 138.525) (end 232.9149 138.4851) (width 0.2) (layer "B.Cu") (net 6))
 (segment (start 248 136) (end 247.2 136) (width 0.2) (layer "F.Cu") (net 8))
 (segment (start 267.21 127.2) (end 265.2 127.2) (width 0.2) (layer "F.Cu") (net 8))
 (segment (start 239.324765 138.024883) (end 239.324765 138.824883) (width 0.2) (layer "F.Cu") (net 8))
 (segment (start 246.4 136.8) (end 240.549648 136.8) (width 0.2) (layer "F.Cu") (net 8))
 (segment (start 238.349648 139.8) (end 236.7199 139.8) (width 0.2) (layer "F.Cu") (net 8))
 (segment (start 265.2 127.2) (end 258.8 133.6) (width 0.2) (layer "F.Cu") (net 8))
 (segment (start 240.549648 136.8) (end 239.324765 138.024883) (width 0.2) (layer "F.Cu") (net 8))
 (segment (start 268.4 126.01) (end 267.21 127.2) (width 0.2) (layer "F.Cu") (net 8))
 (segment (start 236.7199 139.8) (end 235.4549 141.065) (width 0.2) (layer "F.Cu") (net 8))
 (segment (start 250.4 133.6) (end 248 136) (width 0.2) (layer "F.Cu") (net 8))
 (segment (start 258.8 133.6) (end 250.4 133.6) (width 0.2) (layer "F.Cu") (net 8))
 (segment (start 247.2 136) (end 246.4 136.8) (width 0.2) (layer "F.Cu") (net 8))
 (segment (start 239.324765 138.824883) (end 238.349648 139.8) (width 0.2) (layer "F.Cu") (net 8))
 (segment (start 235.4549 141.065) (end 235.4549 141.1549) (width 0.2) (layer "B.Cu") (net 8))
 (segment (start 237.9949 138.5051) (end 237.9949 138.525) (width 0.2) (layer "F.Cu") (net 9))
 (segment (start 237.9949 138.525) (end 238.475 138.525) (width 0.2) (layer "B.Cu") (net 9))
 (segment (start 265.81 126.01) (end 265.86 126.01) (width 0.2) (layer "B.Cu") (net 9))
 (segment (start 248.3 136.4) (end 250.7 134) (width 0.2) (layer "B.Cu") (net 9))
 (segment (start 257.82 134) (end 265.81 126.01) (width 0.2) (layer "B.Cu") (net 9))
 (segment (start 238.475 138.525) (end 240.6 136.4) (width 0.2) (layer "B.Cu") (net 9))
 (segment (start 240.6 136.4) (end 248.3 136.4) (width 0.2) (layer "B.Cu") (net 9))
 (segment (start 250.7 134) (end 257.82 134) (width 0.2) (layer "B.Cu") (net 9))
 (segment (start 243.8 139.8) (end 239.2599 139.8) (width 0.2) (layer "F.Cu") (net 10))
 (segment (start 244.4 137.9) (end 244.4 139.2) (width 0.2) (layer "F.Cu") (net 10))
 (segment (start 265 129.8) (end 260.8 134) (width 0.2) (layer "F.Cu") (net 10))
 (segment (start 244.4 139.2) (end 243.8 139.8) (width 0.2) (layer "F.Cu") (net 10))
 (segment (start 267.15 129.8) (end 265 129.8) (width 0.2) (layer "F.Cu") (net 10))
 (segment (start 260.8 134) (end 250.7 134) (width 0.2) (layer "F.Cu") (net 10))
 (segment (start 245.1 137.2) (end 244.4 137.9) (width 0.2) (layer "F.Cu") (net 10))
 (segment (start 250.7 134) (end 248.3 136.4) (width 0.2) (layer "F.Cu") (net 10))
 (segment (start 239.2599 139.8) (end 237.9949 141.065) (width 0.2) (layer "F.Cu") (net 10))
 (segment (start 246.7 137.2) (end 245.1 137.2) (width 0.2) (layer "F.Cu") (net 10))
 (segment (start 248.3 136.4) (end 247.5 136.4) (width 0.2) (layer "F.Cu") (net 10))
 (segment (start 268.4 128.55) (end 267.15 129.8) (width 0.2) (layer "F.Cu") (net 10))
 (segment (start 247.5 136.4) (end 246.7 137.2) (width 0.2) (layer "F.Cu") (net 10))
 (segment (start 265.719874 128.55) (end 265.86 128.55) (width 0.2) (layer "B.Cu") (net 11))
 (segment (start 241.175 138.525) (end 242.9 136.8) (width 0.2) (layer "B.Cu") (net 11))
 (segment (start 240.5349 138.525) (end 241.175 138.525) (width 0.2) (layer "B.Cu") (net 11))
 (segment (start 251 134.4) (end 259.869874 134.4) (width 0.2) (layer "B.Cu") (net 11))
 (segment (start 259.869874 134.4) (end 265.719874 128.55) (width 0.2) (layer "B.Cu") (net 11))
 (segment (start 265.86 128.55) (end 265.86 128.5) (width 0.2) (layer "B.Cu") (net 11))
 (segment (start 248.6 136.8) (end 251 134.4) (width 0.2) (layer "B.Cu") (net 11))
 (segment (start 242.9 136.8) (end 248.6 136.8) (width 0.2) (layer "B.Cu") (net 11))
 (segment (start 243.0749 138.525) (end 243.075 138.525) (width 0.2) (layer "F.Cu") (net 12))
 (segment (start 244.4 137.2) (end 248.8 137.2) (width 0.2) (layer "B.Cu") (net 12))
 (segment (start 265.2 132.3) (end 267.19 132.3) (width 0.2) (layer "B.Cu") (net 12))
 (segment (start 243.0749 138.525) (end 243.075 138.525) (width 0.2) (layer "B.Cu") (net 12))
 (segment (start 243.075 138.525) (end 244.4 137.2) (width 0.2) (layer "B.Cu") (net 12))
 (segment (start 251.2 134.8) (end 262.7 134.8) (width 0.2) (layer "B.Cu") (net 12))
 (segment (start 262.7 134.8) (end 265.2 132.3) (width 0.2) (layer "B.Cu") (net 12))
 (segment (start 268.4 131.09) (end 268.4 131.04) (width 0.2) (layer "B.Cu") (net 12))
 (segment (start 267.19 132.3) (end 268.4 131.09) (width 0.2) (layer "B.Cu") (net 12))
 (segment (start 248.8 137.2) (end 251.2 134.8) (width 0.2) (layer "B.Cu") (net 12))
 (segment (start 265.86 131.09) (end 265.86 131.04) (width 0.2) (layer "F.Cu") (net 13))
 (segment (start 246.9 137.8) (end 247.9 136.8) (width 0.2) (layer "F.Cu") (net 13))
 (segment (start 243.0749 141.065) (end 243.465 141.065) (width 0.2) (layer "F.Cu") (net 13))
 (segment (start 246.9 139.2) (end 246.9 137.8) (width 0.2) (layer "F.Cu") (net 13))
 (segment (start 246.3 139.8) (end 246.9 139.2) (width 0.2) (layer "F.Cu") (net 13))
 (segment (start 247.9 136.8) (end 248.6 136.8) (width 0.2) (layer "F.Cu") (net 13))
 (segment (start 243.465 141.065) (end 243.5 141.1) (width 0.2) (layer "F.Cu") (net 13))
 (segment (start 244.8 139.8) (end 246.3 139.8) (width 0.2) (layer "F.Cu") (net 13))
 (segment (start 243.0749 141.065) (end 243.1099 141.1) (width 0.2) (layer "F.Cu") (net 13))
 (segment (start 262.55 134.4) (end 265.86 131.09) (width 0.2) (layer "F.Cu") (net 13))
 (segment (start 248.6 136.8) (end 251 134.4) (width 0.2) (layer "F.Cu") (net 13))
 (segment (start 251 134.4) (end 262.55 134.4) (width 0.2) (layer "F.Cu") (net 13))
 (segment (start 243.5 141.1) (end 244.8 139.8) (width 0.2) (layer "F.Cu") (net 13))
 (segment (start 267.23 134.8) (end 268.4 133.63) (width 0.2) (layer "B.Cu") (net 14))
 (segment (start 249.4 137.2) (end 251.4 135.2) (width 0.2) (layer "B.Cu") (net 14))
 (segment (start 245.725 138.525) (end 247 139.8) (width 0.2) (layer "B.Cu") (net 14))
 (segment (start 265.1 134.8) (end 267.23 134.8) (width 0.2) (layer "B.Cu") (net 14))
 (segment (start 251.4 135.2) (end 264.7 135.2) (width 0.2) (layer "B.Cu") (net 14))
 (segment (start 245.6149 138.525) (end 245.725 138.525) (width 0.2) (layer "B.Cu") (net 14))
 (segment (start 264.7 135.2) (end 265.1 134.8) (width 0.2) (layer "B.Cu") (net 14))
 (segment (start 247 139.8) (end 248.9 139.8) (width 0.2) (layer "B.Cu") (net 14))
 (segment (start 268.4 133.63) (end 268.4 133.58) (width 0.2) (layer "B.Cu") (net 14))
 (segment (start 249.4 139.3) (end 249.4 137.2) (width 0.2) (layer "B.Cu") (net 14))
 (segment (start 248.9 139.8) (end 249.4 139.3) (width 0.2) (layer "B.Cu") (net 14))
 (segment (start 268.4 136.12) (end 267.08 134.8) (width 0.2) (layer "F.Cu") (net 15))
 (segment (start 249.8 136.2) (end 248.1549 137.8451) (width 0.2) (layer "F.Cu") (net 15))
 (segment (start 248.1549 137.8451) (end 248.1549 138.525) (width 0.2) (layer "F.Cu") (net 15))
 (segment (start 267.08 134.8) (end 265.1 134.8) (width 0.2) (layer "F.Cu") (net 15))
 (segment (start 265.1 134.8) (end 251.2 134.8) (width 0.2) (layer "F.Cu") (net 15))
 (segment (start 251.2 134.8) (end 249.8 136.2) (width 0.2) (layer "F.Cu") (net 15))
 (segment (start 262.02 136.12) (end 261.8 135.9) (width 0.2) (layer "F.Cu") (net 16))
 (segment (start 265.86 136.12) (end 262.02 136.12) (width 0.2) (layer "F.Cu") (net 16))
 (segment (start 248.1549 141.065) (end 248.1549 141.0451) (width 0.2) (layer "F.Cu") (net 16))
 (segment (start 261.1 135.2) (end 260 135.2) (width 0.2) (layer "F.Cu") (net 16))
 (segment (start 249.4 137.2) (end 251.4 135.2) (width 0.2) (layer "F.Cu") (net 16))
 (segment (start 248.1549 141.0451) (end 249.4 139.8) (width 0.2) (layer "F.Cu") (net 16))
 (segment (start 260 135.2) (end 252.4 135.2) (width 0.2) (layer "F.Cu") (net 16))
 (segment (start 251.4 135.2) (end 252.9 135.2) (width 0.2) (layer "F.Cu") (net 16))
 (segment (start 249.4 139.8) (end 249.4 137.2) (width 0.2) (layer "F.Cu") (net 16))
 (segment (start 261.8 135.9) (end 261.1 135.2) (width 0.2) (layer "F.Cu") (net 16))
 (segment (start 268.4 138.66) (end 268.4 138.71) (width 0.2) (layer "F.Cu") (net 17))
 (segment (start 262.7 137.4) (end 260.9 135.6) (width 0.2) (layer "F.Cu") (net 17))
 (segment (start 268.4 138.7) (end 267.1 137.4) (width 0.2) (layer "F.Cu") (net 17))
 (segment (start 267.1 137.4) (end 262.7 137.4) (width 0.2) (layer "F.Cu") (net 17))
 (segment (start 250.6949 138.4051) (end 250.6949 138.525) (width 0.2) (layer "F.Cu") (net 17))
 (segment (start 268.4 138.71) (end 268.4 138.7) (width 0.2) (layer "F.Cu") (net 17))
 (segment (start 253.5 135.6) (end 250.6949 138.4051) (width 0.2) (layer "F.Cu") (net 17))
 (segment (start 260.9 135.6) (end 253.5 135.6) (width 0.2) (layer "F.Cu") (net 17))
 (segment (start 265.86 138.66) (end 265.86 139.24) (width 0.2) (layer "F.Cu") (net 18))
 (segment (start 250.6949 141.065) (end 250.765 141.065) (width 0.2) (layer "F.Cu") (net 18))
 (segment (start 250.6949 141.065) (end 250.6949 140.5051) (width 0.2) (layer "B.Cu") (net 18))
 (segment (start 254.1 135.6) (end 262.75 135.6) (width 0.2) (layer "B.Cu") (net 18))
 (segment (start 265.81 138.66) (end 265.86 138.66) (width 0.2) (layer "B.Cu") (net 18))
 (segment (start 250.6949 141.065) (end 250.735 141.065) (width 0.2) (layer "B.Cu") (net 18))
 (segment (start 250.6949 140.5051) (end 252 139.2) (width 0.2) (layer "B.Cu") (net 18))
 (segment (start 252 137.7) (end 254.1 135.6) (width 0.2) (layer "B.Cu") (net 18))
 (segment (start 252 139.2) (end 252 137.7) (width 0.2) (layer "B.Cu") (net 18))
 (segment (start 262.75 135.6) (end 265.81 138.66) (width 0.2) (layer "B.Cu") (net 18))
 (segment (start 253.2349 141.065) (end 252 139.8301) (width 0.2) (layer "F.Cu") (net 19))
 (segment (start 265.81 141.2) (end 265.8 141.2) (width 0.2) (layer "F.Cu") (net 19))
 (segment (start 253.7 136) (end 260.61 136) (width 0.2) (layer "F.Cu") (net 19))
 (segment (start 253.2349 141.065) (end 253.265 141.065) (width 0.2) (layer "F.Cu") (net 19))
 (segment (start 260.61 136) (end 265.81 141.2) (width 0.2) (layer "F.Cu") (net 19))
 (segment (start 252 137.7) (end 253.7 136) (width 0.2) (layer "F.Cu") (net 19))
 (segment (start 252 139.8301) (end 252 137.7) (width 0.2) (layer "F.Cu") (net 19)))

